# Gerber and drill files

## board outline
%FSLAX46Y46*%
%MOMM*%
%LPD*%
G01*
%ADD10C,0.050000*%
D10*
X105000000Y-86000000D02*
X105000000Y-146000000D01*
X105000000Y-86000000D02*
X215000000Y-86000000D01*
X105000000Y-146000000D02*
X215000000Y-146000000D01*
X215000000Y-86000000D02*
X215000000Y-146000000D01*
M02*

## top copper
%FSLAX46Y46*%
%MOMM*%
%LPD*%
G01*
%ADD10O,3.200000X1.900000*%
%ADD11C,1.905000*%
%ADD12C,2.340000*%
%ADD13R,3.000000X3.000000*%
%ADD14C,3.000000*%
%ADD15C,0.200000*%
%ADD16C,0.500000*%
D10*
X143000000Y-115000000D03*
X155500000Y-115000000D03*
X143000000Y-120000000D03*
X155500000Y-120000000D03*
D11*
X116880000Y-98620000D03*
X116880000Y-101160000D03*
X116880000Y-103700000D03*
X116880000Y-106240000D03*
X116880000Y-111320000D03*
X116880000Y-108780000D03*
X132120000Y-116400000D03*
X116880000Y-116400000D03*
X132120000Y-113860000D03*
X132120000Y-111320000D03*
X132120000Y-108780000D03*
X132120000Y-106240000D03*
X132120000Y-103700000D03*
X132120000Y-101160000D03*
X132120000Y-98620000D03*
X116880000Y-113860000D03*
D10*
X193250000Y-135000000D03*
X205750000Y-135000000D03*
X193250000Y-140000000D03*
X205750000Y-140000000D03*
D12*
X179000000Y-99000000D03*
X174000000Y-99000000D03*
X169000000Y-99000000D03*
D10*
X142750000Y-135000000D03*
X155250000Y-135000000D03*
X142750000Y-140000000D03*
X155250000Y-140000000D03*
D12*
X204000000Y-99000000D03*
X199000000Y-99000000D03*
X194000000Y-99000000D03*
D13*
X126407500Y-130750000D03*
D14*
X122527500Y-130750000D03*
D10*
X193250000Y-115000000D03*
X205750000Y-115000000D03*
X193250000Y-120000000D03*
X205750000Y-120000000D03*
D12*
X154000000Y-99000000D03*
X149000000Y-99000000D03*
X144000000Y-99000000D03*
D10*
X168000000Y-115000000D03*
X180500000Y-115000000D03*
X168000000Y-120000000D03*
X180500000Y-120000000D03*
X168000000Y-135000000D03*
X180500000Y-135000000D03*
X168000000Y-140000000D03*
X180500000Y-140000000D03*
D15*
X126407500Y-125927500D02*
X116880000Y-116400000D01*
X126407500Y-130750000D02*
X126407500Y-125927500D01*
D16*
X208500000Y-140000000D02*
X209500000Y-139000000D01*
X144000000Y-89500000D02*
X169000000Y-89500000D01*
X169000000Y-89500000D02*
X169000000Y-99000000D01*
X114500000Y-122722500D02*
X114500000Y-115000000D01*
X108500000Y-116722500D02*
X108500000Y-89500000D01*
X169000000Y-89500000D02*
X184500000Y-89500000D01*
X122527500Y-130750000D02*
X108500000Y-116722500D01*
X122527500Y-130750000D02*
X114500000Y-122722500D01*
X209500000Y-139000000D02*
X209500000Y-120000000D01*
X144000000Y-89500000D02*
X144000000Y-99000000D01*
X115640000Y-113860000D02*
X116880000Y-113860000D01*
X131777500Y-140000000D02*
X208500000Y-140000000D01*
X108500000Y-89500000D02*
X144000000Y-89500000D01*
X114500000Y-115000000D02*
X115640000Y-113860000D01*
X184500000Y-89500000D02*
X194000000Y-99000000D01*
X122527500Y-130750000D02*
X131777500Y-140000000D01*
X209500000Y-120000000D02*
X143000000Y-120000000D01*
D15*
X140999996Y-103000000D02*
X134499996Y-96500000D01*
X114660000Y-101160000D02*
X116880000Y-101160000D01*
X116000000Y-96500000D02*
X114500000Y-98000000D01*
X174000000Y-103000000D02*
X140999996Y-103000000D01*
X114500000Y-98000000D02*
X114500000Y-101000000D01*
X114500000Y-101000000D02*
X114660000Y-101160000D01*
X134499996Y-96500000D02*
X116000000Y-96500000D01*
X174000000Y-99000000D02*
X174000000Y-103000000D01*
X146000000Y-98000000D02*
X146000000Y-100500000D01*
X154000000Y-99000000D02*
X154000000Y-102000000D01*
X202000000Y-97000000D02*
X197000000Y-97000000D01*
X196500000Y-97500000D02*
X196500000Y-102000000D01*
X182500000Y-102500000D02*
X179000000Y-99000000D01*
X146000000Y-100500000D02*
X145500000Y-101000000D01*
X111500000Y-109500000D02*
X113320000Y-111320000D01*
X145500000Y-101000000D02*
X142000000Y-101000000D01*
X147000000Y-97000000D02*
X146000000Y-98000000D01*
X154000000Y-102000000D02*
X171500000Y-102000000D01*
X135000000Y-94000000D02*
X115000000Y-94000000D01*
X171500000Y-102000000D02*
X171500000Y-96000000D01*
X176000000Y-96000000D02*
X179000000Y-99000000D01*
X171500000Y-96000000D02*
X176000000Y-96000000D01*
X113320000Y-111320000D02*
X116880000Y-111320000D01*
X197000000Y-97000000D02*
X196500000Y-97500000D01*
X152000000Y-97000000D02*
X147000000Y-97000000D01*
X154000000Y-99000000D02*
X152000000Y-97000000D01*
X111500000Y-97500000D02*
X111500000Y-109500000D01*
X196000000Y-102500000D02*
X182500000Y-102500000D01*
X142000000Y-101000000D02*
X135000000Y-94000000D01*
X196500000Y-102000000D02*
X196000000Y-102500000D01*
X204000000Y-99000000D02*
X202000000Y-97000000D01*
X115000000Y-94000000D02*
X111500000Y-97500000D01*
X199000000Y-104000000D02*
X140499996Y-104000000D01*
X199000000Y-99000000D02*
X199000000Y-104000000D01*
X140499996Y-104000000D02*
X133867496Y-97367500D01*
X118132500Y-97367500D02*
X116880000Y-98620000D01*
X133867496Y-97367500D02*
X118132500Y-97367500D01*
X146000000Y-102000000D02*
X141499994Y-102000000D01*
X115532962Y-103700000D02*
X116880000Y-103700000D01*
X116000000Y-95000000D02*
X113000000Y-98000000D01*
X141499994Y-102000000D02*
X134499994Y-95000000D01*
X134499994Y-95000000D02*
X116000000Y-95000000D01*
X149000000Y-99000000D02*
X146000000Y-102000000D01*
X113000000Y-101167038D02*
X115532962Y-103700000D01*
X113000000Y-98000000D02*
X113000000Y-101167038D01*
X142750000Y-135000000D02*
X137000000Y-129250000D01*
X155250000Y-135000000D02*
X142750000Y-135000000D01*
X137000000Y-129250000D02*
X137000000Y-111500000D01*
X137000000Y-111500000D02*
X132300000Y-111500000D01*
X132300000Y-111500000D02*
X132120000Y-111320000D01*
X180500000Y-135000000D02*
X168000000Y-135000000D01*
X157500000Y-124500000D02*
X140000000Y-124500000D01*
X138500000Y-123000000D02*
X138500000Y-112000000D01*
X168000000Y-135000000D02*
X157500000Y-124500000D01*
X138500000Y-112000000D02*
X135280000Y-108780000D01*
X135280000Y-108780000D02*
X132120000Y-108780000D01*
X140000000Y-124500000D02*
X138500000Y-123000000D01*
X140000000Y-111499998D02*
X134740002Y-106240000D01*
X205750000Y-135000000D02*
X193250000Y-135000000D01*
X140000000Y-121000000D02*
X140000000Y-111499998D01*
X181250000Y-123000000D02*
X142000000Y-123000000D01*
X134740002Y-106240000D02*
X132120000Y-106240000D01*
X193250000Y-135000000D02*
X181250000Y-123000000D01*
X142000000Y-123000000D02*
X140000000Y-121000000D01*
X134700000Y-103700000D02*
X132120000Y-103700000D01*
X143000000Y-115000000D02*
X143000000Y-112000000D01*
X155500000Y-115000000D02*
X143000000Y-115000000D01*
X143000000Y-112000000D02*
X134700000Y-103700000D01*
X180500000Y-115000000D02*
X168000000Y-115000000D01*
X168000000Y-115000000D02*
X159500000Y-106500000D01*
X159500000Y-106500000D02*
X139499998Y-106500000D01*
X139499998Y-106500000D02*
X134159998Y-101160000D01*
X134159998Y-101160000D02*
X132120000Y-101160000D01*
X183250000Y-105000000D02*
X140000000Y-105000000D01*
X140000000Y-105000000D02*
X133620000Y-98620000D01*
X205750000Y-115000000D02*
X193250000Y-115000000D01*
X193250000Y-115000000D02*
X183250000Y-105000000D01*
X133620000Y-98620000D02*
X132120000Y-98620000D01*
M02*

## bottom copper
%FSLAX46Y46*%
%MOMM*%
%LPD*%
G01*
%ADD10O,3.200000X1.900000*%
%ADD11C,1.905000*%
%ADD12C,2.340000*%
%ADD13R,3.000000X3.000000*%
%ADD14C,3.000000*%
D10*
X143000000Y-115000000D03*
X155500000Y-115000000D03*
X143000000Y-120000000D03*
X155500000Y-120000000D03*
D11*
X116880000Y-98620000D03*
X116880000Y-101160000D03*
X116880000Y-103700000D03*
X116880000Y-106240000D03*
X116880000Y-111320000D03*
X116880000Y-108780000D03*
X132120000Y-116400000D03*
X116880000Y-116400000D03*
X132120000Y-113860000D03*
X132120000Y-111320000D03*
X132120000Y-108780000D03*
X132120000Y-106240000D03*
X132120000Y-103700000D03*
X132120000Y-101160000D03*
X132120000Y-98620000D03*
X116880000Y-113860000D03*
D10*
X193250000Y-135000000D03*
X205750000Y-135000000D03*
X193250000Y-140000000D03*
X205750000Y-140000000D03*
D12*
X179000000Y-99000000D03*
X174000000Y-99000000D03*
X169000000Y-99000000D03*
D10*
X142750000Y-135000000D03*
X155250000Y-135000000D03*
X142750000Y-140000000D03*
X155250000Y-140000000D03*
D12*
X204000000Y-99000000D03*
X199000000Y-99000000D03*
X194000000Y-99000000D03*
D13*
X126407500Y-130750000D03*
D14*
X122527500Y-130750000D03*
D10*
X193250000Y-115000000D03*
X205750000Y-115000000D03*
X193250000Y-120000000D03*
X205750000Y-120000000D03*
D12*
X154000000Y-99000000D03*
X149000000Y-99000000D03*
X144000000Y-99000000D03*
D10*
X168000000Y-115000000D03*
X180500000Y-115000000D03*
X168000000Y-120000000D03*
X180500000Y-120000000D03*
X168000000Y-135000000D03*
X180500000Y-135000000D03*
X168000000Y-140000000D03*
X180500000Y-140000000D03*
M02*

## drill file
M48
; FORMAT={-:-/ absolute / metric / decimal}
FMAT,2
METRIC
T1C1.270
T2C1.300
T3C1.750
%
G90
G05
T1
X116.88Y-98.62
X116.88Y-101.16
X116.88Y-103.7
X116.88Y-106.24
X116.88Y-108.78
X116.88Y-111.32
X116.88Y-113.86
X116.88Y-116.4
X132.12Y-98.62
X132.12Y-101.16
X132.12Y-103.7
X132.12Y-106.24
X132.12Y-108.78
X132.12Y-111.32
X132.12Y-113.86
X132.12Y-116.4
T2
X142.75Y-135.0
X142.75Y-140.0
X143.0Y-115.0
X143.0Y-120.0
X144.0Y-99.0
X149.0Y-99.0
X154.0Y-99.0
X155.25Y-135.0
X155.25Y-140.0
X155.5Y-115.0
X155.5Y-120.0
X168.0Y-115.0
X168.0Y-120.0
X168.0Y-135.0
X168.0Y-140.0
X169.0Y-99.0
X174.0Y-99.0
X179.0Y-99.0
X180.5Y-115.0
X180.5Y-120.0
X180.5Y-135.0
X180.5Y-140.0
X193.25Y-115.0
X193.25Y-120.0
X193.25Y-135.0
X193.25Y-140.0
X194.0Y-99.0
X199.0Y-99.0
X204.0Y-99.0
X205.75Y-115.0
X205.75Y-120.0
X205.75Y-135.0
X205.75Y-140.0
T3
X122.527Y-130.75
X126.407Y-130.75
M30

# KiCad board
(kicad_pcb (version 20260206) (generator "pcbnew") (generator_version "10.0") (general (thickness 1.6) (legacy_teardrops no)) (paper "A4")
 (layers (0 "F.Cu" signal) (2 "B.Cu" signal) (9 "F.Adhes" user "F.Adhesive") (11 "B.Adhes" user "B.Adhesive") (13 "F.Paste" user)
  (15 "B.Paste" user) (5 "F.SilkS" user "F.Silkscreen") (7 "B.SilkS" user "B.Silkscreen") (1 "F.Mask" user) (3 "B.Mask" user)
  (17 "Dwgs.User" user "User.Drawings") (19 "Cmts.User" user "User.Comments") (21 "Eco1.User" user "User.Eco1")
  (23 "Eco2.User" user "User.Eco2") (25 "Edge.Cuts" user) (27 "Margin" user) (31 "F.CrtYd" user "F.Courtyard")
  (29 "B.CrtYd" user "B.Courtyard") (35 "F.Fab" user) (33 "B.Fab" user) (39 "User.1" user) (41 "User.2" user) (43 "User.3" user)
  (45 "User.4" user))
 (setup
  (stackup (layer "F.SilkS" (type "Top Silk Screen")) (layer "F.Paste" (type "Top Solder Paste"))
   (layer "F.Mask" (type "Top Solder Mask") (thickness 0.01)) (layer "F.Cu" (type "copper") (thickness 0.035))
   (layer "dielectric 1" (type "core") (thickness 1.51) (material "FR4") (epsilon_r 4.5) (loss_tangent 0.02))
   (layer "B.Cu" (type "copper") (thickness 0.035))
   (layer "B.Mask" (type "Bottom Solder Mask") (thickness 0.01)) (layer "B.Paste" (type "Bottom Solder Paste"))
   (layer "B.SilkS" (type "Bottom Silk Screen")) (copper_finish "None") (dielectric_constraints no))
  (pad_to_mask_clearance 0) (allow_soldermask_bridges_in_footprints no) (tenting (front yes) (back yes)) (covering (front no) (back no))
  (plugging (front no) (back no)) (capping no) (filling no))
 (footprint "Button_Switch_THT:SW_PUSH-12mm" (layer "F.Cu") (at 143 115)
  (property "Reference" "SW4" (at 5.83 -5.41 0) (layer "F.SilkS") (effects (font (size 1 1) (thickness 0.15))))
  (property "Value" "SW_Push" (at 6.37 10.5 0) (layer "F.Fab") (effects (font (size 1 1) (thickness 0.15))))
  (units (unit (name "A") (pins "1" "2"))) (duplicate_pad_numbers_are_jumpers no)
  (pad "1" thru_hole oval (at 0 0) (size 3.2 1.9) (drill 1.3) (layers "*.Cu" "*.Mask") (remove_unused_layers no) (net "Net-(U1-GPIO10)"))
  (pad "1" thru_hole oval (at 12.5 0) (size 3.2 1.9) (drill 1.3) (layers "*.Cu" "*.Mask") (remove_unused_layers no) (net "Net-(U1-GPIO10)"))
  (pad "2" thru_hole oval (at 0 5) (size 3.2 1.9) (drill 1.3) (layers "*.Cu" "*.Mask") (remove_unused_layers no) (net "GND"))
  (pad "2" thru_hole oval (at 12.5 5) (size 3.2 1.9) (drill 1.3) (layers "*.Cu" "*.Mask") (remove_unused_layers no) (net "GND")))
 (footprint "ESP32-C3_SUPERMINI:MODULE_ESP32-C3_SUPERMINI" (layer "F.Cu") (at 124.5 106.5 180)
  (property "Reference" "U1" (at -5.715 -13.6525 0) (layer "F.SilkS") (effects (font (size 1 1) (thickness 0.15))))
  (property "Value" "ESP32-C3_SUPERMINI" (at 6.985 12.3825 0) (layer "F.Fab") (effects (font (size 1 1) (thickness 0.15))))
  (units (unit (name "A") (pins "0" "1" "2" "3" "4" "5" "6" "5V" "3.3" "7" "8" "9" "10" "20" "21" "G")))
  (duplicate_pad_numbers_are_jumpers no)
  (pad "0" thru_hole circle (at 7.62 7.88 180) (size 1.905 1.905) (drill 1.27) (layers "*.Cu" "*.Mask") (remove_unused_layers no)
   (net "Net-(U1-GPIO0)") (solder_mask_margin 0.102))
  (pad "1" thru_hole circle (at 7.62 5.34 180) (size 1.905 1.905) (drill 1.27) (layers "*.Cu" "*.Mask") (remove_unused_layers no)
   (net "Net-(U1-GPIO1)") (solder_mask_margin 0.102))
  (pad "2" thru_hole circle (at 7.62 2.8 180) (size 1.905 1.905) (drill 1.27) (layers "*.Cu" "*.Mask") (remove_unused_layers no)
   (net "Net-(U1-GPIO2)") (solder_mask_margin 0.102))
  (pad "3" thru_hole circle (at 7.62 0.26 180) (size 1.905 1.905) (drill 1.27) (layers "*.Cu" "*.Mask") (remove_unused_layers no)
   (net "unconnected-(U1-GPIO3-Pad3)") (solder_mask_margin 0.102))
  (pad "3.3" thru_hole circle (at 7.62 -4.82 180) (size 1.905 1.905) (drill 1.27) (layers "*.Cu" "*.Mask") (remove_unused_layers no)
   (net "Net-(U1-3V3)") (solder_mask_margin 0.102))
  (pad "4" thru_hole circle (at 7.62 -2.28 180) (size 1.905 1.905) (drill 1.27) (layers "*.Cu" "*.Mask") (remove_unused_layers no)
   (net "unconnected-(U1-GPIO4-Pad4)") (solder_mask_margin 0.102))
  (pad "5" thru_hole circle (at -7.62 -9.9 180) (size 1.905 1.905) (drill 1.27) (layers "*.Cu" "*.Mask") (remove_unused_layers no)
   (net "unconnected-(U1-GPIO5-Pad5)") (solder_mask_margin 0.102))
  (pad "5V" thru_hole circle (at 7.62 -9.9 180) (size 1.905 1.905) (drill 1.27) (layers "*.Cu" "*.Mask") (remove_unused_layers no)
   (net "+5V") (solder_mask_margin 0.102))
  (pad "6" thru_hole circle (at -7.62 -7.36 180) (size 1.905 1.905) (drill 1.27) (layers "*.Cu" "*.Mask") (remove_unused_layers no)
   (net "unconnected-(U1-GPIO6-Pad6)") (solder_mask_margin 0.102))
  (pad "7" thru_hole circle (at -7.62 -4.82 180) (size 1.905 1.905) (drill 1.27) (layers "*.Cu" "*.Mask") (remove_unused_layers no)
   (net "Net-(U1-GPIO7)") (solder_mask_margin 0.102))
  (pad "8" thru_hole circle (at -7.62 -2.28 180) (size 1.905 1.905) (drill 1.27) (layers "*.Cu" "*.Mask") (remove_unused_layers no)
   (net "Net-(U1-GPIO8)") (solder_mask_margin 0.102))
  (pad "9" thru_hole circle (at -7.62 0.26 180) (size 1.905 1.905) (drill 1.27) (layers "*.Cu" "*.Mask") (remove_unused_layers no)
   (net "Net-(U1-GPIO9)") (solder_mask_margin 0.102))
  (pad "10" thru_hole circle (at -7.62 2.8 180) (size 1.905 1.905) (drill 1.27) (layers "*.Cu" "*.Mask") (remove_unused_layers no)
   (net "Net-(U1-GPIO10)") (solder_mask_margin 0.102))
  (pad "20" thru_hole circle (at -7.62 5.34 180) (size 1.905 1.905) (drill 1.27) (layers "*.Cu" "*.Mask") (remove_unused_layers no)
   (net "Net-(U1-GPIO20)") (solder_mask_margin 0.102))
  (pad "21" thru_hole circle (at -7.62 7.88 180) (size 1.905 1.905) (drill 1.27) (layers "*.Cu" "*.Mask") (remove_unused_layers no)
   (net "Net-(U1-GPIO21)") (solder_mask_margin 0.102))
  (pad "G" thru_hole circle (at 7.62 -7.36 180) (size 1.905 1.905) (drill 1.27) (layers "*.Cu" "*.Mask") (remove_unused_layers no)
   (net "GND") (solder_mask_margin 0.102)))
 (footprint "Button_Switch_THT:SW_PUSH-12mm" (layer "F.Cu") (at 193.25 135)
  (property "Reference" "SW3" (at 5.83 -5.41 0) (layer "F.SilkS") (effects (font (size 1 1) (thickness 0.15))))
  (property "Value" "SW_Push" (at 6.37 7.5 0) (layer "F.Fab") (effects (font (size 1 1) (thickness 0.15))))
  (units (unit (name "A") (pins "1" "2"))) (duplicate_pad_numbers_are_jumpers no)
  (pad "1" thru_hole oval (at 0 0) (size 3.2 1.9) (drill 1.3) (layers "*.Cu" "*.Mask") (remove_unused_layers no) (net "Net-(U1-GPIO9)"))
  (pad "1" thru_hole oval (at 12.5 0) (size 3.2 1.9) (drill 1.3) (layers "*.Cu" "*.Mask") (remove_unused_layers no) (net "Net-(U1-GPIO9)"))
  (pad "2" thru_hole oval (at 0 5) (size 3.2 1.9) (drill 1.3) (layers "*.Cu" "*.Mask") (remove_unused_layers no) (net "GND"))
  (pad "2" thru_hole oval (at 12.5 5) (size 3.2 1.9) (drill 1.3) (layers "*.Cu" "*.Mask") (remove_unused_layers no) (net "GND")))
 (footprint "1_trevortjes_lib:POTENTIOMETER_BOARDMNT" (layer "F.Cu") (at 179 99 90)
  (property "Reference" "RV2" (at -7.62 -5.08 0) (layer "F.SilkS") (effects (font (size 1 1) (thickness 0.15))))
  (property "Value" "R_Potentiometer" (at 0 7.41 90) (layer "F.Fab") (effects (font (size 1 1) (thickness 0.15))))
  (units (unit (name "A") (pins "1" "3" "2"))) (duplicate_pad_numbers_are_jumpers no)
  (pad "1" thru_hole circle (at 0 0 90) (size 2.34 2.34) (drill 1.3) (layers "*.Cu" "*.Mask") (remove_unused_layers no) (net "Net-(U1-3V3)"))
  (pad "2" thru_hole circle (at 0 -5 90) (size 2.34 2.34) (drill 1.3) (layers "*.Cu" "*.Mask") (remove_unused_layers no)
   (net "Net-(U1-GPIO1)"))
  (pad "3" thru_hole circle (at 0 -10 90) (size 2.34 2.34) (drill 1.3) (layers "*.Cu" "*.Mask") (remove_unused_layers no) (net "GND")))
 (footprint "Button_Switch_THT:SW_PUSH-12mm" (layer "F.Cu") (at 142.75 135)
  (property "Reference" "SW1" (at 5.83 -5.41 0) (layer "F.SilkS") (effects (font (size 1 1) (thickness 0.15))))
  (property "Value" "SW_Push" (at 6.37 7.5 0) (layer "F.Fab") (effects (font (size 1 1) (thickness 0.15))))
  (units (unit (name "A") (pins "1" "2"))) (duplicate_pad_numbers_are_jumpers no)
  (pad "1" thru_hole oval (at 0 0) (size 3.2 1.9) (drill 1.3) (layers "*.Cu" "*.Mask") (remove_unused_layers no) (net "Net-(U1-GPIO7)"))
  (pad "1" thru_hole oval (at 12.5 0) (size 3.2 1.9) (drill 1.3) (layers "*.Cu" "*.Mask") (remove_unused_layers no) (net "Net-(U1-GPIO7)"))
  (pad "2" thru_hole oval (at 0 5) (size 3.2 1.9) (drill 1.3) (layers "*.Cu" "*.Mask") (remove_unused_layers no) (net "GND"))
  (pad "2" thru_hole oval (at 12.5 5) (size 3.2 1.9) (drill 1.3) (layers "*.Cu" "*.Mask") (remove_unused_layers no) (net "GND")))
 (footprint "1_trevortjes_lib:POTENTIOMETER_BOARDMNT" (layer "F.Cu") (at 204 99 90)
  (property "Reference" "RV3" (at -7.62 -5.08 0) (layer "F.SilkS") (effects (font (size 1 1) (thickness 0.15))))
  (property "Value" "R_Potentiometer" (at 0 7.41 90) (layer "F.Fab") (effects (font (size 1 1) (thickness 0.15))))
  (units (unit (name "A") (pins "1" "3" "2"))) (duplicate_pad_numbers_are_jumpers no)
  (pad "1" thru_hole circle (at 0 0 90) (size 2.34 2.34) (drill 1.3) (layers "*.Cu" "*.Mask") (remove_unused_layers no) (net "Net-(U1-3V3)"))
  (pad "2" thru_hole circle (at 0 -5 90) (size 2.34 2.34) (drill 1.3) (layers "*.Cu" "*.Mask") (remove_unused_layers no)
   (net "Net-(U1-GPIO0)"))
  (pad "3" thru_hole circle (at 0 -10 90) (size 2.34 2.34) (drill 1.3) (layers "*.Cu" "*.Mask") (remove_unused_layers no) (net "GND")))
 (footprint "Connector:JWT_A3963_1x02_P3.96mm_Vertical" (layer "F.Cu") (at 126.4075 130.75 180)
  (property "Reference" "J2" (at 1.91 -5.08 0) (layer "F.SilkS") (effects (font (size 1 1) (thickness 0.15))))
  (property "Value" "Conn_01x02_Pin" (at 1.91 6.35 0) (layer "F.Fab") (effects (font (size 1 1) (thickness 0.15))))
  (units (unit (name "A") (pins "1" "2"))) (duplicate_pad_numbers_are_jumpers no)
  (pad "1" thru_hole rect (at 0 0 180) (size 3 3) (drill 1.75) (layers "*.Cu" "*.Mask") (remove_unused_layers no) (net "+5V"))
  (pad "2" thru_hole circle (at 3.88 0 180) (size 3 3) (drill 1.75) (layers "*.Cu" "*.Mask") (remove_unused_layers no) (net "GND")))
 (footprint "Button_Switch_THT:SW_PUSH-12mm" (layer "F.Cu") (at 193.25 115)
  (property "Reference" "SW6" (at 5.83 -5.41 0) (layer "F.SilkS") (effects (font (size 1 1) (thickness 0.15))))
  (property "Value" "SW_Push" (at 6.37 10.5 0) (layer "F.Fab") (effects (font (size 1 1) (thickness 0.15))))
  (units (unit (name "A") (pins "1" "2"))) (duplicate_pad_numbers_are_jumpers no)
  (pad "1" thru_hole oval (at 0 0) (size 3.2 1.9) (drill 1.3) (layers "*.Cu" "*.Mask") (remove_unused_layers no) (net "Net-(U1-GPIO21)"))
  (pad "1" thru_hole oval (at 12.5 0) (size 3.2 1.9) (drill 1.3) (layers "*.Cu" "*.Mask") (remove_unused_layers no) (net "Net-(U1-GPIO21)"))
  (pad "2" thru_hole oval (at 0 5) (size 3.2 1.9) (drill 1.3) (layers "*.Cu" "*.Mask") (remove_unused_layers no) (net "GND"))
  (pad "2" thru_hole oval (at 12.5 5) (size 3.2 1.9) (drill 1.3) (layers "*.Cu" "*.Mask") (remove_unused_layers no) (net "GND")))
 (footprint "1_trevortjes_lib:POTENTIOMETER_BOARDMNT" (layer "F.Cu") (at 154 99 90)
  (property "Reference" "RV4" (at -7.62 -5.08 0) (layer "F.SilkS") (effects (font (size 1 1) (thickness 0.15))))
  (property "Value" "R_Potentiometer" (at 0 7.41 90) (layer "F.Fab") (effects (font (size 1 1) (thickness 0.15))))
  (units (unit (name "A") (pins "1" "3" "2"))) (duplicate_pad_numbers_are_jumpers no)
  (pad "1" thru_hole circle (at 0 0 90) (size 2.34 2.34) (drill 1.3) (layers "*.Cu" "*.Mask") (remove_unused_layers no) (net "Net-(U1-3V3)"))
  (pad "2" thru_hole circle (at 0 -5 90) (size 2.34 2.34) (drill 1.3) (layers "*.Cu" "*.Mask") (remove_unused_layers no)
   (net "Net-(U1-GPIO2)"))
  (pad "3" thru_hole circle (at 0 -10 90) (size 2.34 2.34) (drill 1.3) (layers "*.Cu" "*.Mask") (remove_unused_layers no) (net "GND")))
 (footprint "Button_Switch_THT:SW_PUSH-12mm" (layer "F.Cu") (at 168 115)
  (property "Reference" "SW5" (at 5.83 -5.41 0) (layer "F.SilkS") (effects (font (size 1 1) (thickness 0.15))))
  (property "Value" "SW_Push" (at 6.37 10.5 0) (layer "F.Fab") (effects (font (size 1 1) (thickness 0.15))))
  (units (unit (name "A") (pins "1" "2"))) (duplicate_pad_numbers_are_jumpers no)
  (pad "1" thru_hole oval (at 0 0) (size 3.2 1.9) (drill 1.3) (layers "*.Cu" "*.Mask") (remove_unused_layers no) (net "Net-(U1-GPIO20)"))
  (pad "1" thru_hole oval (at 12.5 0) (size 3.2 1.9) (drill 1.3) (layers "*.Cu" "*.Mask") (remove_unused_layers no) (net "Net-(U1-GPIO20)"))
  (pad "2" thru_hole oval (at 0 5) (size 3.2 1.9) (drill 1.3) (layers "*.Cu" "*.Mask") (remove_unused_layers no) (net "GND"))
  (pad "2" thru_hole oval (at 12.5 5) (size 3.2 1.9) (drill 1.3) (layers "*.Cu" "*.Mask") (remove_unused_layers no) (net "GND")))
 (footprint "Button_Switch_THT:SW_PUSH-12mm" (layer "F.Cu") (at 168 135)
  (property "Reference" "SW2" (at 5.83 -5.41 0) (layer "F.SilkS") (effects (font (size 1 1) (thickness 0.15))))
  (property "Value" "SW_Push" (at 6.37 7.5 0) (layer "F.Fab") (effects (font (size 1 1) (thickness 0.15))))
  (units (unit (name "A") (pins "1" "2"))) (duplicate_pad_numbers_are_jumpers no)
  (pad "1" thru_hole oval (at 0 0) (size 3.2 1.9) (drill 1.3) (layers "*.Cu" "*.Mask") (remove_unused_layers no) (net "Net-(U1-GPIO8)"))
  (pad "1" thru_hole oval (at 12.5 0) (size 3.2 1.9) (drill 1.3) (layers "*.Cu" "*.Mask") (remove_unused_layers no) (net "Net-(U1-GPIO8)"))
  (pad "2" thru_hole oval (at 0 5) (size 3.2 1.9) (drill 1.3) (layers "*.Cu" "*.Mask") (remove_unused_layers no) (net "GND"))
  (pad "2" thru_hole oval (at 12.5 5) (size 3.2 1.9) (drill 1.3) (layers "*.Cu" "*.Mask") (remove_unused_layers no) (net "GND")))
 (gr_line (start 105 86) (end 105 146) (stroke (width 0.05) (type default)) (layer "Edge.Cuts"))
 (gr_line (start 105 86) (end 215 86) (stroke (width 0.05) (type default)) (layer "Edge.Cuts"))
 (gr_line (start 105 146) (end 215 146) (stroke (width 0.05) (type default)) (layer "Edge.Cuts"))
 (gr_line (start 215 86) (end 215 146) (stroke (width 0.05) (type default)) (layer "Edge.Cuts"))
 (segment (start 126.4075 125.9275) (end 116.88 116.4) (width 0.2) (layer "F.Cu") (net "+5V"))
 (segment (start 126.4075 130.75) (end 126.4075 125.9275) (width 0.2) (layer "F.Cu") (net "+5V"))
 (segment (start 208.5 140) (end 209.5 139) (width 0.5) (layer "F.Cu") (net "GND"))
 (segment (start 144 89.5) (end 169 89.5) (width 0.5) (layer "F.Cu") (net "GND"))
 (segment (start 169 89.5) (end 169 99) (width 0.5) (layer "F.Cu") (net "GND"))
 (segment (start 114.5 122.7225) (end 114.5 115) (width 0.5) (layer "F.Cu") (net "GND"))
 (segment (start 108.5 116.7225) (end 108.5 89.5) (width 0.5) (layer "F.Cu") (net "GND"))
 (segment (start 169 89.5) (end 184.5 89.5) (width 0.5) (layer "F.Cu") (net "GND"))
 (segment (start 122.5275 130.75) (end 108.5 116.7225) (width 0.5) (layer "F.Cu") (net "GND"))
 (segment (start 122.5275 130.75) (end 114.5 122.7225) (width 0.5) (layer "F.Cu") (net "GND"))
 (segment (start 209.5 139) (end 209.5 120) (width 0.5) (layer "F.Cu") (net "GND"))
 (segment (start 144 89.5) (end 144 99) (width 0.5) (layer "F.Cu") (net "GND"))
 (segment (start 115.64 113.86) (end 116.88 113.86) (width 0.5) (layer "F.Cu") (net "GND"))
 (segment (start 131.7775 140) (end 208.5 140) (width 0.5) (layer "F.Cu") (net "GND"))
 (segment (start 108.5 89.5) (end 144 89.5) (width 0.5) (layer "F.Cu") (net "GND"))
 (segment (start 114.5 115) (end 115.64 113.86) (width 0.5) (layer "F.Cu") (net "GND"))
 (segment (start 184.5 89.5) (end 194 99) (width 0.5) (layer "F.Cu") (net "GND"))
 (segment (start 122.5275 130.75) (end 131.7775 140) (width 0.5) (layer "F.Cu") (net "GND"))
 (segment (start 209.5 120) (end 143 120) (width 0.5) (layer "F.Cu") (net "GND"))
 (segment (start 140.999996 103) (end 134.499996 96.5) (width 0.2) (layer "F.Cu") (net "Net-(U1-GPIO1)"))
 (segment (start 114.66 101.16) (end 116.88 101.16) (width 0.2) (layer "F.Cu") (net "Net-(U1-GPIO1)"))
 (segment (start 116 96.5) (end 114.5 98) (width 0.2) (layer "F.Cu") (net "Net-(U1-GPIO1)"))
 (segment (start 174 103) (end 140.999996 103) (width 0.2) (layer "F.Cu") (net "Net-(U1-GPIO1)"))
 (segment (start 114.5 98) (end 114.5 101) (width 0.2) (layer "F.Cu") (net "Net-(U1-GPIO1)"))
 (segment (start 114.5 101) (end 114.66 101.16) (width 0.2) (layer "F.Cu") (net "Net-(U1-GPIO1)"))
 (segment (start 134.499996 96.5) (end 116 96.5) (width 0.2) (layer "F.Cu") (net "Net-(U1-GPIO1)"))
 (segment (start 174 99) (end 174 103) (width 0.2) (layer "F.Cu") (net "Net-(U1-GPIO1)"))
 (segment (start 146 98) (end 146 100.5) (width 0.2) (layer "F.Cu") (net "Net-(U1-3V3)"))
 (segment (start 154 99) (end 154 102) (width 0.2) (layer "F.Cu") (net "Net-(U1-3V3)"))
 (segment (start 202 97) (end 197 97) (width 0.2) (layer "F.Cu") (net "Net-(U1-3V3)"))
 (segment (start 196.5 97.5) (end 196.5 102) (width 0.2) (layer "F.Cu") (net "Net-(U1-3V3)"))
 (segment (start 182.5 102.5) (end 179 99) (width 0.2) (layer "F.Cu") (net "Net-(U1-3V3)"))
 (segment (start 146 100.5) (end 145.5 101) (width 0.2) (layer "F.Cu") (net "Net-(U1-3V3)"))
 (segment (start 111.5 109.5) (end 113.32 111.32) (width 0.2) (layer "F.Cu") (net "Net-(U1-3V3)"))
 (segment (start 145.5 101) (end 142 101) (width 0.2) (layer "F.Cu") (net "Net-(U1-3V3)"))
 (segment (start 147 97) (end 146 98) (width 0.2) (layer "F.Cu") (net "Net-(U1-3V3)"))
 (segment (start 154 102) (end 171.5 102) (width 0.2) (layer "F.Cu") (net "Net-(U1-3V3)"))
 (segment (start 135 94) (end 115 94) (width 0.2) (layer "F.Cu") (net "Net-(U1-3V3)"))
 (segment (start 171.5 102) (end 171.5 96) (width 0.2) (layer "F.Cu") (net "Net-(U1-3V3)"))
 (segment (start 176 96) (end 179 99) (width 0.2) (layer "F.Cu") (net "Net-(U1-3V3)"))
 (segment (start 171.5 96) (end 176 96) (width 0.2) (layer "F.Cu") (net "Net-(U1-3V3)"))
 (segment (start 113.32 111.32) (end 116.88 111.32) (width 0.2) (layer "F.Cu") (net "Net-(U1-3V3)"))
 (segment (start 197 97) (end 196.5 97.5) (width 0.2) (layer "F.Cu") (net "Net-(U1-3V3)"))
 (segment (start 152 97) (end 147 97) (width 0.2) (layer "F.Cu") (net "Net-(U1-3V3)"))
 (segment (start 154 99) (end 152 97) (width 0.2) (layer "F.Cu") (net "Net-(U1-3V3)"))
 (segment (start 111.5 97.5) (end 111.5 109.5) (width 0.2) (layer "F.Cu") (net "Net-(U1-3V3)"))
 (segment (start 196 102.5) (end 182.5 102.5) (width 0.2) (layer "F.Cu") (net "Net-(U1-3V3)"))
 (segment (start 142 101) (end 135 94) (width 0.2) (layer "F.Cu") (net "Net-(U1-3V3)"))
 (segment (start 196.5 102) (end 196 102.5) (width 0.2) (layer "F.Cu") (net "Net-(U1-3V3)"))
 (segment (start 204 99) (end 202 97) (width 0.2) (layer "F.Cu") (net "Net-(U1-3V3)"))
 (segment (start 115 94) (end 111.5 97.5) (width 0.2) (layer "F.Cu") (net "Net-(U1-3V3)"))
 (segment (start 199 104) (end 140.499996 104) (width 0.2) (layer "F.Cu") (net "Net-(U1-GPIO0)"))
 (segment (start 199 99) (end 199 104) (width 0.2) (layer "F.Cu") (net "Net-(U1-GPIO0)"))
 (segment (start 140.499996 104) (end 133.867496 97.3675) (width 0.2) (layer "F.Cu") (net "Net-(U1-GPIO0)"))
 (segment (start 118.1325 97.3675) (end 116.88 98.62) (width 0.2) (layer "F.Cu") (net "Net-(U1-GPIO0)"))
 (segment (start 133.867496 97.3675) (end 118.1325 97.3675) (width 0.2) (layer "F.Cu") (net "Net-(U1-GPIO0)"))
 (segment (start 146 102) (end 141.499994 102) (width 0.2) (layer "F.Cu") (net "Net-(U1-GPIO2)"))
 (segment (start 115.532962 103.7) (end 116.88 103.7) (width 0.2) (layer "F.Cu") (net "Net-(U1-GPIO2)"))
 (segment (start 116 95) (end 113 98) (width 0.2) (layer "F.Cu") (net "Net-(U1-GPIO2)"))
 (segment (start 141.499994 102) (end 134.499994 95) (width 0.2) (layer "F.Cu") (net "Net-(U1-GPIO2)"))
 (segment (start 134.499994 95) (end 116 95) (width 0.2) (layer "F.Cu") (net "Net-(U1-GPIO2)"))
 (segment (start 149 99) (end 146 102) (width 0.2) (layer "F.Cu") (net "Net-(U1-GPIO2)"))
 (segment (start 113 101.167038) (end 115.532962 103.7) (width 0.2) (layer "F.Cu") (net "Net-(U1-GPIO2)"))
 (segment (start 113 98) (end 113 101.167038) (width 0.2) (layer "F.Cu") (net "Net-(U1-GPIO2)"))
 (segment (start 142.75 135) (end 137 129.25) (width 0.2) (layer "F.Cu") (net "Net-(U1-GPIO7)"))
 (segment (start 155.25 135) (end 142.75 135) (width 0.2) (layer "F.Cu") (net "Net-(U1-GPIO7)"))
 (segment (start 137 129.25) (end 137 111.5) (width 0.2) (layer "F.Cu") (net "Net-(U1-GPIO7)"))
 (segment (start 137 111.5) (end 132.3 111.5) (width 0.2) (layer "F.Cu") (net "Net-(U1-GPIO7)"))
 (segment (start 132.3 111.5) (end 132.12 111.32) (width 0.2) (layer "F.Cu") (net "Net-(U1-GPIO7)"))
 (segment (start 180.5 135) (end 168 135) (width 0.2) (layer "F.Cu") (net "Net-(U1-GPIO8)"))
 (segment (start 157.5 124.5) (end 140 124.5) (width 0.2) (layer "F.Cu") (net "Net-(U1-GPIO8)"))
 (segment (start 138.5 123) (end 138.5 112) (width 0.2) (layer "F.Cu") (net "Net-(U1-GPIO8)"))
 (segment (start 168 135) (end 157.5 124.5) (width 0.2) (layer "F.Cu") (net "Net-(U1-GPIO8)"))
 (segment (start 138.5 112) (end 135.28 108.78) (width 0.2) (layer "F.Cu") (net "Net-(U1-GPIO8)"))
 (segment (start 135.28 108.78) (end 132.12 108.78) (width 0.2) (layer "F.Cu") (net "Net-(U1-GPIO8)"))
 (segment (start 140 124.5) (end 138.5 123) (width 0.2) (layer "F.Cu") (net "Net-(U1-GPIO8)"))
 (segment (start 140 111.499998) (end 134.740002 106.24) (width 0.2) (layer "F.Cu") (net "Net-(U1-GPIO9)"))
 (segment (start 205.75 135) (end 193.25 135) (width 0.2) (layer "F.Cu") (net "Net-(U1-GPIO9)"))
 (segment (start 140 121) (end 140 111.499998) (width 0.2) (layer "F.Cu") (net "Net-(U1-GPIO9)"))
 (segment (start 181.25 123) (end 142 123) (width 0.2) (layer "F.Cu") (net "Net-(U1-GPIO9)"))
 (segment (start 134.740002 106.24) (end 132.12 106.24) (width 0.2) (layer "F.Cu") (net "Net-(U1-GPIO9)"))
 (segment (start 193.25 135) (end 181.25 123) (width 0.2) (layer "F.Cu") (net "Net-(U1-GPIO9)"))
 (segment (start 142 123) (end 140 121) (width 0.2) (layer "F.Cu") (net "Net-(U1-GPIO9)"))
 (segment (start 134.7 103.7) (end 132.12 103.7) (width 0.2) (layer "F.Cu") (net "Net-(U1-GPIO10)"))
 (segment (start 143 115) (end 143 112) (width 0.2) (layer "F.Cu") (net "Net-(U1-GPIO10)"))
 (segment (start 155.5 115) (end 143 115) (width 0.2) (layer "F.Cu") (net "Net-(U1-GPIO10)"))
 (segment (start 143 112) (end 134.7 103.7) (width 0.2) (layer "F.Cu") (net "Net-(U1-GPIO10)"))
 (segment (start 180.5 115) (end 168 115) (width 0.2) (layer "F.Cu") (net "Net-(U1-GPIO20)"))
 (segment (start 168 115) (end 159.5 106.5) (width 0.2) (layer "F.Cu") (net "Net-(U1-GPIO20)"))
 (segment (start 159.5 106.5) (end 139.499998 106.5) (width 0.2) (layer "F.Cu") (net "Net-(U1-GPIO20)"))
 (segment (start 139.499998 106.5) (end 134.159998 101.16) (width 0.2) (layer "F.Cu") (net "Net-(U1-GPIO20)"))
 (segment (start 134.159998 101.16) (end 132.12 101.16) (width 0.2) (layer "F.Cu") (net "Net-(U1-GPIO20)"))
 (segment (start 183.25 105) (end 140 105) (width 0.2) (layer "F.Cu") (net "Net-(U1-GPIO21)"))
 (segment (start 140 105) (end 133.62 98.62) (width 0.2) (layer "F.Cu") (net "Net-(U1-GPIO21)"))
 (segment (start 205.75 115) (end 193.25 115) (width 0.2) (layer "F.Cu") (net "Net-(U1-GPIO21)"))
 (segment (start 193.25 115) (end 183.25 105) (width 0.2) (layer "F.Cu") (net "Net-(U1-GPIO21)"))
 (segment (start 133.62 98.62) (end 132.12 98.62) (width 0.2) (layer "F.Cu") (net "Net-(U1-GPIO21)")))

